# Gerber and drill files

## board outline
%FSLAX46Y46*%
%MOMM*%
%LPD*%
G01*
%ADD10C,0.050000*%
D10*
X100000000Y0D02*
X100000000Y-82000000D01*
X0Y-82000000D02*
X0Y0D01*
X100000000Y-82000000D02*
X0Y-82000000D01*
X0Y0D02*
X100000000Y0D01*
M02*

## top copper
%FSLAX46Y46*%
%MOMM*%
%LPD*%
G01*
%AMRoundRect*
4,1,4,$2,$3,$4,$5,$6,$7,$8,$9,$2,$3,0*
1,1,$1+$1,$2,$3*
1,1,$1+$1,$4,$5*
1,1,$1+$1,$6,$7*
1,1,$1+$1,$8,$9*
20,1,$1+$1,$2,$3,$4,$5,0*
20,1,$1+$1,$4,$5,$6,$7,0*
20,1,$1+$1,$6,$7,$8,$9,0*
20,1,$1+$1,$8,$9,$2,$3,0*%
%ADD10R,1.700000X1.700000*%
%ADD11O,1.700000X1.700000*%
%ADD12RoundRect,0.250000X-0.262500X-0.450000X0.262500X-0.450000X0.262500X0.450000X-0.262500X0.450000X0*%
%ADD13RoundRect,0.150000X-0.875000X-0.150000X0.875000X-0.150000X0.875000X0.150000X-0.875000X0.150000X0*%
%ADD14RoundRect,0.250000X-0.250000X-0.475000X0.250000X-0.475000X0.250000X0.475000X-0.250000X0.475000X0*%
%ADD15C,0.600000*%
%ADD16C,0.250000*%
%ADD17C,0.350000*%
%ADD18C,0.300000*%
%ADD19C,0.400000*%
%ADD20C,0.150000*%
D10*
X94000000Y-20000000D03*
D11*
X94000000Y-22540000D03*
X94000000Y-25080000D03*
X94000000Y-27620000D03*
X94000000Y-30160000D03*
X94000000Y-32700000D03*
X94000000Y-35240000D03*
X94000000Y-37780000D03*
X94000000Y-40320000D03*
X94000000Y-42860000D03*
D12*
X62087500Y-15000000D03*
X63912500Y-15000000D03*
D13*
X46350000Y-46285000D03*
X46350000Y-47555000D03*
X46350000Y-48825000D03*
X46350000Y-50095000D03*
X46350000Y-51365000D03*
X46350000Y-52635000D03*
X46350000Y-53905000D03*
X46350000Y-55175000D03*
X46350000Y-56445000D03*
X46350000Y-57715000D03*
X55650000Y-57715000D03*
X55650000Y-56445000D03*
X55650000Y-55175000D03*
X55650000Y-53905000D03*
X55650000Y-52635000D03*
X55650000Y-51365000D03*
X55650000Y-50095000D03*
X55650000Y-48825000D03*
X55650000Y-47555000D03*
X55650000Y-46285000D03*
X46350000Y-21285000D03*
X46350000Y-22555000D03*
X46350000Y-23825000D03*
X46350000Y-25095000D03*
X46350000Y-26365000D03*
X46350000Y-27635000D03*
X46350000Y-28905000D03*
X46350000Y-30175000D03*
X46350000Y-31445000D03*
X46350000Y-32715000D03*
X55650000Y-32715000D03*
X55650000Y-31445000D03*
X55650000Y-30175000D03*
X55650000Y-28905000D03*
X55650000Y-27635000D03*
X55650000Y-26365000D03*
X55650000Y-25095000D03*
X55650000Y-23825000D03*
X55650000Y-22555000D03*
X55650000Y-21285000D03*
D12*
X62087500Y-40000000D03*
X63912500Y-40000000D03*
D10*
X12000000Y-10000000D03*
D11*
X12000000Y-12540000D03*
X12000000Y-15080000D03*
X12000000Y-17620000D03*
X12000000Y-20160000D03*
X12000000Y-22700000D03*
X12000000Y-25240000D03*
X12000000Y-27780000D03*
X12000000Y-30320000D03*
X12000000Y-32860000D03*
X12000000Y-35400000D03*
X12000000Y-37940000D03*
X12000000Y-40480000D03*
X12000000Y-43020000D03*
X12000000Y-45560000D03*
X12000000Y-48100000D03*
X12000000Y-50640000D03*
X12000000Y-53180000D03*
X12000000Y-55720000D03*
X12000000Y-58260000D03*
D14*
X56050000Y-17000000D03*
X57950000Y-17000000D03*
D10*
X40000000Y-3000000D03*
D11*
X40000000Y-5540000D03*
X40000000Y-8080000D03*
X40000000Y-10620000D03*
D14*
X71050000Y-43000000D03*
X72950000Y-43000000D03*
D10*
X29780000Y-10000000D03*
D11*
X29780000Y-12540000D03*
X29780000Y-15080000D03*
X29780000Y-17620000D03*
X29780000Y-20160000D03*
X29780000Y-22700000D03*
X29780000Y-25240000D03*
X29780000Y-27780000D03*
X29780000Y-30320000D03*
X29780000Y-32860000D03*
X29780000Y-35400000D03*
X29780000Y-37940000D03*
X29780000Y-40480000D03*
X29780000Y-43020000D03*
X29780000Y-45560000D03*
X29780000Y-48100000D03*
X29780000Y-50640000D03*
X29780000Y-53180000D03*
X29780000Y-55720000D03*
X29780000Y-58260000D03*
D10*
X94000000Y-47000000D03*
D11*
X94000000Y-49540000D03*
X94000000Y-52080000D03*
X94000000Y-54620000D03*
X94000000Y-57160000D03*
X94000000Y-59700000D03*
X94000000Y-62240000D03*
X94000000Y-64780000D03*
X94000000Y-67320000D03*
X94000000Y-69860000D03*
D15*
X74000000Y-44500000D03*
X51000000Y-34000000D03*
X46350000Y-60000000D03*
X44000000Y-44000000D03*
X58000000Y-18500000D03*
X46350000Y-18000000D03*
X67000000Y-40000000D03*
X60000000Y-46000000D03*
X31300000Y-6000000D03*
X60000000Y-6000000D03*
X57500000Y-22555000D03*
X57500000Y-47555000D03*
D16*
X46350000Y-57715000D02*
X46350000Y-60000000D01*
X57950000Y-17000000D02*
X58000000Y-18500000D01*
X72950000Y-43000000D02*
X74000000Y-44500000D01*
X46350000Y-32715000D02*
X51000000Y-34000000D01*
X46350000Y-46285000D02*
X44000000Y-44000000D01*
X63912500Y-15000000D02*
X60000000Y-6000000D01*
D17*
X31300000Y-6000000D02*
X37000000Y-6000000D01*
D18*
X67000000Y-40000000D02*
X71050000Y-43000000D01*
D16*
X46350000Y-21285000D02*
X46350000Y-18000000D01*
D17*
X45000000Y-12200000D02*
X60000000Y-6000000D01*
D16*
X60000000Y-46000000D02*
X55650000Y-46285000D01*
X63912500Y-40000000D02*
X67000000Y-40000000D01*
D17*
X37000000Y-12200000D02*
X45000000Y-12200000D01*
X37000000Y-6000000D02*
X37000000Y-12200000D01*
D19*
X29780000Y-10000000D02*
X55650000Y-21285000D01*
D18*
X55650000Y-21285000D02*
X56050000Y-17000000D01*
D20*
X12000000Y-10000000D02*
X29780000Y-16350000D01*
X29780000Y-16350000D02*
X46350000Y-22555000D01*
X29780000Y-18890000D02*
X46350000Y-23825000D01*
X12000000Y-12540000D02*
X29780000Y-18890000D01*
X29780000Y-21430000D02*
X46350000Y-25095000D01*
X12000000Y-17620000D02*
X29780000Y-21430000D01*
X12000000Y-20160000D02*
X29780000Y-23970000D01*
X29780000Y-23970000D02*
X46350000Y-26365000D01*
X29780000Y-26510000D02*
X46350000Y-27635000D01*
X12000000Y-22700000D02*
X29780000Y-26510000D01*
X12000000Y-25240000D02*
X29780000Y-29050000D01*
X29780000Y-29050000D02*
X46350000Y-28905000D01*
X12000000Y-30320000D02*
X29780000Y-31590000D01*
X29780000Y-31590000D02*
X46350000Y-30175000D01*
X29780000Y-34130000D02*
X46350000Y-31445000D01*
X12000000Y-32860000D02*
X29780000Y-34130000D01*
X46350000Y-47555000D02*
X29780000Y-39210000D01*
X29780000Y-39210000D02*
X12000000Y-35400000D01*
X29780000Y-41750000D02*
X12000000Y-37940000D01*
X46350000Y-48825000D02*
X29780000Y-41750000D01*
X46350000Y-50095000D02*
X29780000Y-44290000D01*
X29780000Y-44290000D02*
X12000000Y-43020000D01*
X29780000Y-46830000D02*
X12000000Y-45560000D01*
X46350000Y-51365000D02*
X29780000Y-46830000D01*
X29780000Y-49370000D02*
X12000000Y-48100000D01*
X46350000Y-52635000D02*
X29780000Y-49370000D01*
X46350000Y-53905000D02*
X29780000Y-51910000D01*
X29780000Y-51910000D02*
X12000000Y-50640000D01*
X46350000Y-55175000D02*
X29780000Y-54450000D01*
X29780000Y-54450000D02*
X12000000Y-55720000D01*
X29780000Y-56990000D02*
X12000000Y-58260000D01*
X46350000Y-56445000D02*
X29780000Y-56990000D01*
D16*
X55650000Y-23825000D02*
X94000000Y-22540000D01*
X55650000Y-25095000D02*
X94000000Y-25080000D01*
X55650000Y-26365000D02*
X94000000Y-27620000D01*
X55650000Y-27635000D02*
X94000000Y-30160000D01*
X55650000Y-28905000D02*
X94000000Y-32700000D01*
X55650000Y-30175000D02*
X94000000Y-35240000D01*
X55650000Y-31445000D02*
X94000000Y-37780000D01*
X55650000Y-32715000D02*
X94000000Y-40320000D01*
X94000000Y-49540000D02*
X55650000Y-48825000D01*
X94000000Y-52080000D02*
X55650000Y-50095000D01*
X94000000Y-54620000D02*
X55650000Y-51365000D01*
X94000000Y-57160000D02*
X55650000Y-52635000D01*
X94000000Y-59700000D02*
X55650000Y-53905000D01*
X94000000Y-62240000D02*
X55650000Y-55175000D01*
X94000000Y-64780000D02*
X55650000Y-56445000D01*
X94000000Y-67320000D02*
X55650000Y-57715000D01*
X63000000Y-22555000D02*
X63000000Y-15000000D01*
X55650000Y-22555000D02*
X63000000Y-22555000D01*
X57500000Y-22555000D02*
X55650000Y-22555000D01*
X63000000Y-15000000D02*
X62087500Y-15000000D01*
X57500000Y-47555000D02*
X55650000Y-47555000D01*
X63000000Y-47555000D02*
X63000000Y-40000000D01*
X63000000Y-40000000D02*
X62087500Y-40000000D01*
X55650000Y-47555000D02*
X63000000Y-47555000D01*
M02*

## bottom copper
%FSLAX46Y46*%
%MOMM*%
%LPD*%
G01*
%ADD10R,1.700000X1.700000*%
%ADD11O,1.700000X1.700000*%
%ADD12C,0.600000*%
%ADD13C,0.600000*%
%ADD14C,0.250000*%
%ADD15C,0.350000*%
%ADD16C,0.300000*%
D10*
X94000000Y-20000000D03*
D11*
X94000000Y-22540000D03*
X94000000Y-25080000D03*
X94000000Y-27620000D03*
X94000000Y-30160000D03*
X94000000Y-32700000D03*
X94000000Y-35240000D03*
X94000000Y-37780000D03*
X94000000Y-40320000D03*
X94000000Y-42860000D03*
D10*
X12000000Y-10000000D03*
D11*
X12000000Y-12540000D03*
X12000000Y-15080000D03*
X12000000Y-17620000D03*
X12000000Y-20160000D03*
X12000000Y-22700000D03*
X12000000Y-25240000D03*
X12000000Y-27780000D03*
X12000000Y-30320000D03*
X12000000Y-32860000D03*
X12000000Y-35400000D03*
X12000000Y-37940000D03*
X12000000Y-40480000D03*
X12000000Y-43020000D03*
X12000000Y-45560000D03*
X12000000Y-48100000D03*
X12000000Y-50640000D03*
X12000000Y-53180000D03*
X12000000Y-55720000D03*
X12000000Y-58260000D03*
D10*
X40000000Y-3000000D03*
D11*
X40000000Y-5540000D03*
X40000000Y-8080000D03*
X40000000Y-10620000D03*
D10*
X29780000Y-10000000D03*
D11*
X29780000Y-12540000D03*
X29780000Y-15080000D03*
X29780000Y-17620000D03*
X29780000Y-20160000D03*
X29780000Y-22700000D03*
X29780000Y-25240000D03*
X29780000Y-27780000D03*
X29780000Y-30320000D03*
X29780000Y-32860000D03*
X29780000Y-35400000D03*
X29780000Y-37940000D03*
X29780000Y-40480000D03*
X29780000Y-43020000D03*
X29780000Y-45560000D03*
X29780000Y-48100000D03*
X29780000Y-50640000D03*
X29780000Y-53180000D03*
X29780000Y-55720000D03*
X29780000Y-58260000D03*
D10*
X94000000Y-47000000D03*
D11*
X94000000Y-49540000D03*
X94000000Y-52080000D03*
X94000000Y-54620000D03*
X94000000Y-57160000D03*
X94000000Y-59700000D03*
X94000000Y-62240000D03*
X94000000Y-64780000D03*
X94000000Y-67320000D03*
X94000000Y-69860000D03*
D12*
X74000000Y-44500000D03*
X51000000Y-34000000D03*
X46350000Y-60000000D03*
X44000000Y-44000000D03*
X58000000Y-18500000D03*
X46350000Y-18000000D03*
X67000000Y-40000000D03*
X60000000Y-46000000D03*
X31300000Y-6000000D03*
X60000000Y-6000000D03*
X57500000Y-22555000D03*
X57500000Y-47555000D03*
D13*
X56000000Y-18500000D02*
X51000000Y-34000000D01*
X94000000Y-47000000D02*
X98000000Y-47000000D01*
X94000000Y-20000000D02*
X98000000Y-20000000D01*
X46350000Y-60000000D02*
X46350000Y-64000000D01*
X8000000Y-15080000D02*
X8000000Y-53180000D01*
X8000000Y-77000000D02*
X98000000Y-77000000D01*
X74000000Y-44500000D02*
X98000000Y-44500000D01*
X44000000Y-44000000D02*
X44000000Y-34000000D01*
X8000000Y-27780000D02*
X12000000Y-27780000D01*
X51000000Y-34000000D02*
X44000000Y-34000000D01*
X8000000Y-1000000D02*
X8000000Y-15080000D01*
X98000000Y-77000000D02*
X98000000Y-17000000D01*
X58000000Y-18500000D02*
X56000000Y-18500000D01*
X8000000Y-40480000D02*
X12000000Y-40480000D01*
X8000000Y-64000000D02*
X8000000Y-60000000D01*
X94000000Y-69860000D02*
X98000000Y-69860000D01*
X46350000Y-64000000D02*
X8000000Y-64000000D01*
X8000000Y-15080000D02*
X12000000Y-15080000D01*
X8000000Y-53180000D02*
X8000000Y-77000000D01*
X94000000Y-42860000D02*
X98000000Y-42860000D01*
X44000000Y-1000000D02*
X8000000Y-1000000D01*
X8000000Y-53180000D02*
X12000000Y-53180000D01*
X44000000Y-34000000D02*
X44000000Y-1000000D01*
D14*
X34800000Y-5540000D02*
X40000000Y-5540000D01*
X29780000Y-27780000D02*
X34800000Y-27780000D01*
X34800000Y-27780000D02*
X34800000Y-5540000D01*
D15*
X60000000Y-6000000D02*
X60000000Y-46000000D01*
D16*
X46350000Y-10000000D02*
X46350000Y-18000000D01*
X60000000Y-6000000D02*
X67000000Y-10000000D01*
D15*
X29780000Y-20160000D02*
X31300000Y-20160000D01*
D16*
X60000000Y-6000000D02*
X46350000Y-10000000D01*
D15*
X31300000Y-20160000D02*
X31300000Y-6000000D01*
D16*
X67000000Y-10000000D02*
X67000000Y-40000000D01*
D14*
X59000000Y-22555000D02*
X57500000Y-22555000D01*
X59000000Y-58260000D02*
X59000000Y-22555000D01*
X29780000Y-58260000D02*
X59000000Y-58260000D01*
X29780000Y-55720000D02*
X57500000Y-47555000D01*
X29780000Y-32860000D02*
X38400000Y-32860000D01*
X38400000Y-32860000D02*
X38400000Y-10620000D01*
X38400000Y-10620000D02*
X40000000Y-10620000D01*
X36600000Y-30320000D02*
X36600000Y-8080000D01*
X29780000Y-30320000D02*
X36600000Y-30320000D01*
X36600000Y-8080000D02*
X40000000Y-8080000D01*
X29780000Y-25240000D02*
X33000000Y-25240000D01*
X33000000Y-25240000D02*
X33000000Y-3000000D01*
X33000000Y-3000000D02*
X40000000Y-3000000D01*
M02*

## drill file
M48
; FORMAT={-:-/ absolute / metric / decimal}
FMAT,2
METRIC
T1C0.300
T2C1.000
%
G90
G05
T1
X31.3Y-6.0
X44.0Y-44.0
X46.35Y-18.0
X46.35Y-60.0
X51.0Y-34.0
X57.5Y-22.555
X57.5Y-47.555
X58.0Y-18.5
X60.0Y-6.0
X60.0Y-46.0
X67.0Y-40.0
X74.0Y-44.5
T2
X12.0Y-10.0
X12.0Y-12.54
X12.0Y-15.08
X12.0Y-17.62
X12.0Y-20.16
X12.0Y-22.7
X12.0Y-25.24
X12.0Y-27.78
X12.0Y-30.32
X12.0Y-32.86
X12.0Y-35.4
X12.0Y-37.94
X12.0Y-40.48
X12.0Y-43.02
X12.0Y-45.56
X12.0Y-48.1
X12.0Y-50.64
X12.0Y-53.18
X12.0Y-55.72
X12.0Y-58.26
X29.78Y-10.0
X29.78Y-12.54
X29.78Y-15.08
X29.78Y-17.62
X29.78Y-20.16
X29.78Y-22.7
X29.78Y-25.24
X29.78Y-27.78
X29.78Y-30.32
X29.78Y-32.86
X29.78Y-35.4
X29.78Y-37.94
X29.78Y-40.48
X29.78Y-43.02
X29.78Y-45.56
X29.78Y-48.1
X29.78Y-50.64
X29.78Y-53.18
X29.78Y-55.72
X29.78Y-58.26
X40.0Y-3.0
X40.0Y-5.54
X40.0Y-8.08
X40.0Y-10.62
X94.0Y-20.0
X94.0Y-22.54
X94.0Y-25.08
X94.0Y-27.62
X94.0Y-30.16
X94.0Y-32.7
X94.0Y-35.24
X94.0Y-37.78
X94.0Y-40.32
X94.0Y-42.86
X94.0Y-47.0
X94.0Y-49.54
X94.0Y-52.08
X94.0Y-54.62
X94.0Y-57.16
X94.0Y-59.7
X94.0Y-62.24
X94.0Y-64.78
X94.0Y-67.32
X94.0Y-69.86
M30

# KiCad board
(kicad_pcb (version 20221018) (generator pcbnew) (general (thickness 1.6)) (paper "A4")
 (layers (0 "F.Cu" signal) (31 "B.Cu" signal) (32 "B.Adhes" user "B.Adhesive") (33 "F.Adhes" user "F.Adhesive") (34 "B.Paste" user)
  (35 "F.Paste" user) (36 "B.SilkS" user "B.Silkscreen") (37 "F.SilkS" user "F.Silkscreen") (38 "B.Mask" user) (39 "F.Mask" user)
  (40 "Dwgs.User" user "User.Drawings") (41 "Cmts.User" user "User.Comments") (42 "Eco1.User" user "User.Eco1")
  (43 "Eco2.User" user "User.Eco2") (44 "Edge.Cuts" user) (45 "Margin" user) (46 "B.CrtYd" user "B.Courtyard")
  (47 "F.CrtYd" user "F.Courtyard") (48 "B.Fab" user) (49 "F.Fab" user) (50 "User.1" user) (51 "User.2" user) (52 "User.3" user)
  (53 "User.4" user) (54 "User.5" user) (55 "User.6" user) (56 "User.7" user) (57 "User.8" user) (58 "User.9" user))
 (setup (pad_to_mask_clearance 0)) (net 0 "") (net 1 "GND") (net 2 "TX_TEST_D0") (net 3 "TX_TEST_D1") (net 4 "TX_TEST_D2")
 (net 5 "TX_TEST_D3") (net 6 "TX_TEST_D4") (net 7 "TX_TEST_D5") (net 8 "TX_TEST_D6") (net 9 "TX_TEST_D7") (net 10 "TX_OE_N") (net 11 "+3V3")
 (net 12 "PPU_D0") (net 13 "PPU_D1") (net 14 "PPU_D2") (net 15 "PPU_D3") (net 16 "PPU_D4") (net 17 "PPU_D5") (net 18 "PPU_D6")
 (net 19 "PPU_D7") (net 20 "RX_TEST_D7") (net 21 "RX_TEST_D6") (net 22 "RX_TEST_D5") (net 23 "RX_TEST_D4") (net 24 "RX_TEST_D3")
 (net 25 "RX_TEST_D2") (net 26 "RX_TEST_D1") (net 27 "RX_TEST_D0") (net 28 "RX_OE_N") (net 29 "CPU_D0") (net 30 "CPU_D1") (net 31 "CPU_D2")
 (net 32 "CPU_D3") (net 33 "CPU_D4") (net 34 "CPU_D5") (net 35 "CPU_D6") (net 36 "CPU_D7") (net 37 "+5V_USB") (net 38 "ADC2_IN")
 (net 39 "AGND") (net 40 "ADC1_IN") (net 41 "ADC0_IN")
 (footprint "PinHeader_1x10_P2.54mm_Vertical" (layer "F.Cu") (at 94 20)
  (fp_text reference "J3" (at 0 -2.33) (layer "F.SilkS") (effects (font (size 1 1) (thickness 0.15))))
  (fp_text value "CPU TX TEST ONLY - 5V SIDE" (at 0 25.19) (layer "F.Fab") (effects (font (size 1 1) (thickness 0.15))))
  (pad "1" thru_hole rect (at 0 0) (size 1.7 1.7) (drill 1) (layers "*.Cu" "*.Mask") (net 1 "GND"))
  (pad "2" thru_hole oval (at 0 2.54) (size 1.7 1.7) (drill 1) (layers "*.Cu" "*.Mask") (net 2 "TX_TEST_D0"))
  (pad "3" thru_hole oval (at 0 5.08) (size 1.7 1.7) (drill 1) (layers "*.Cu" "*.Mask") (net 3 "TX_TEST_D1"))
  (pad "4" thru_hole oval (at 0 7.62) (size 1.7 1.7) (drill 1) (layers "*.Cu" "*.Mask") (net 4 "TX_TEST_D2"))
  (pad "5" thru_hole oval (at 0 10.16) (size 1.7 1.7) (drill 1) (layers "*.Cu" "*.Mask") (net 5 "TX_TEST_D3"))
  (pad "6" thru_hole oval (at 0 12.7) (size 1.7 1.7) (drill 1) (layers "*.Cu" "*.Mask") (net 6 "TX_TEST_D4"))
  (pad "7" thru_hole oval (at 0 15.24) (size 1.7 1.7) (drill 1) (layers "*.Cu" "*.Mask") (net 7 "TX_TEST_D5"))
  (pad "8" thru_hole oval (at 0 17.78) (size 1.7 1.7) (drill 1) (layers "*.Cu" "*.Mask") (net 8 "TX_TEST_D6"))
  (pad "9" thru_hole oval (at 0 20.32) (size 1.7 1.7) (drill 1) (layers "*.Cu" "*.Mask") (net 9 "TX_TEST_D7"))
  (pad "10" thru_hole oval (at 0 22.86) (size 1.7 1.7) (drill 1) (layers "*.Cu" "*.Mask") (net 1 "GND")))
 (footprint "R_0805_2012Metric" (layer "F.Cu") (at 63 15)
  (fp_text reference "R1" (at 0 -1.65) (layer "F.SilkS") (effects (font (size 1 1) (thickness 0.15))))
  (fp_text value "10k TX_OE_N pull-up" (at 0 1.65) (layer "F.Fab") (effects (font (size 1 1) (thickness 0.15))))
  (pad "1" smd roundrect (at -0.9125 0) (size 1.025 1.4) (layers "F.Cu" "F.Paste" "F.Mask") (roundrect_rratio 0.243902) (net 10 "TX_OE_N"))
  (pad "2" smd roundrect (at 0.9125 0) (size 1.025 1.4) (layers "F.Cu" "F.Paste" "F.Mask") (roundrect_rratio 0.243902) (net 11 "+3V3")))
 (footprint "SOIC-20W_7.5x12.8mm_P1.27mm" (layer "F.Cu") (at 51 52)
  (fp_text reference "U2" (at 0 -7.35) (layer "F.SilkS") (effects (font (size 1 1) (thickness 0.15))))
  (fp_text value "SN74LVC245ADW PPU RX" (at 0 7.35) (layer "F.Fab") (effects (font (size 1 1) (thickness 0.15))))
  (pad "1" smd roundrect (at -4.65 -5.715) (size 2.05 0.6) (layers "F.Cu" "F.Paste" "F.Mask") (roundrect_rratio 0.25) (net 1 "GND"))
  (pad "2" smd roundrect (at -4.65 -4.445) (size 2.05 0.6) (layers "F.Cu" "F.Paste" "F.Mask") (roundrect_rratio 0.25) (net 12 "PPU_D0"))
  (pad "3" smd roundrect (at -4.65 -3.175) (size 2.05 0.6) (layers "F.Cu" "F.Paste" "F.Mask") (roundrect_rratio 0.25) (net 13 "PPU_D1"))
  (pad "4" smd roundrect (at -4.65 -1.905) (size 2.05 0.6) (layers "F.Cu" "F.Paste" "F.Mask") (roundrect_rratio 0.25) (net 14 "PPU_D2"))
  (pad "5" smd roundrect (at -4.65 -0.635) (size 2.05 0.6) (layers "F.Cu" "F.Paste" "F.Mask") (roundrect_rratio 0.25) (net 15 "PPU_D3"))
  (pad "6" smd roundrect (at -4.65 0.635) (size 2.05 0.6) (layers "F.Cu" "F.Paste" "F.Mask") (roundrect_rratio 0.25) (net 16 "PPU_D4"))
  (pad "7" smd roundrect (at -4.65 1.905) (size 2.05 0.6) (layers "F.Cu" "F.Paste" "F.Mask") (roundrect_rratio 0.25) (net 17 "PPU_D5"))
  (pad "8" smd roundrect (at -4.65 3.175) (size 2.05 0.6) (layers "F.Cu" "F.Paste" "F.Mask") (roundrect_rratio 0.25) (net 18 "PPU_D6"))
  (pad "9" smd roundrect (at -4.65 4.445) (size 2.05 0.6) (layers "F.Cu" "F.Paste" "F.Mask") (roundrect_rratio 0.25) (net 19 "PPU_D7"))
  (pad "10" smd roundrect (at -4.65 5.715) (size 2.05 0.6) (layers "F.Cu" "F.Paste" "F.Mask") (roundrect_rratio 0.25) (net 1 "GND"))
  (pad "11" smd roundrect (at 4.65 5.715) (size 2.05 0.6) (layers "F.Cu" "F.Paste" "F.Mask") (roundrect_rratio 0.25) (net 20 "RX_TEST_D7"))
  (pad "12" smd roundrect (at 4.65 4.445) (size 2.05 0.6) (layers "F.Cu" "F.Paste" "F.Mask") (roundrect_rratio 0.25) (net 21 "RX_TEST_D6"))
  (pad "13" smd roundrect (at 4.65 3.175) (size 2.05 0.6) (layers "F.Cu" "F.Paste" "F.Mask") (roundrect_rratio 0.25) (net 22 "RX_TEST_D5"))
  (pad "14" smd roundrect (at 4.65 1.905) (size 2.05 0.6) (layers "F.Cu" "F.Paste" "F.Mask") (roundrect_rratio 0.25) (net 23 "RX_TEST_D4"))
  (pad "15" smd roundrect (at 4.65 0.635) (size 2.05 0.6) (layers "F.Cu" "F.Paste" "F.Mask") (roundrect_rratio 0.25) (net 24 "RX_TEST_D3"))
  (pad "16" smd roundrect (at 4.65 -0.635) (size 2.05 0.6) (layers "F.Cu" "F.Paste" "F.Mask") (roundrect_rratio 0.25) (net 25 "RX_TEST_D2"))
  (pad "17" smd roundrect (at 4.65 -1.905) (size 2.05 0.6) (layers "F.Cu" "F.Paste" "F.Mask") (roundrect_rratio 0.25) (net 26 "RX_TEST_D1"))
  (pad "18" smd roundrect (at 4.65 -3.175) (size 2.05 0.6) (layers "F.Cu" "F.Paste" "F.Mask") (roundrect_rratio 0.25) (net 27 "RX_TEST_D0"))
  (pad "19" smd roundrect (at 4.65 -4.445) (size 2.05 0.6) (layers "F.Cu" "F.Paste" "F.Mask") (roundrect_rratio 0.25) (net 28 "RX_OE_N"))
  (pad "20" smd roundrect (at 4.65 -5.715) (size 2.05 0.6) (layers "F.Cu" "F.Paste" "F.Mask") (roundrect_rratio 0.25) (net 11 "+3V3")))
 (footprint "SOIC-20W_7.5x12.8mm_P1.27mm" (layer "F.Cu") (at 51 27)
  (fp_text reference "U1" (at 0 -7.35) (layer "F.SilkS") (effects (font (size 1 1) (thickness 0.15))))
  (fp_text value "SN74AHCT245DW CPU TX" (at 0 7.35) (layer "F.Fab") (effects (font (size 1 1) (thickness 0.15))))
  (pad "1" smd roundrect (at -4.65 -5.715) (size 2.05 0.6) (layers "F.Cu" "F.Paste" "F.Mask") (roundrect_rratio 0.25) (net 11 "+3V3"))
  (pad "2" smd roundrect (at -4.65 -4.445) (size 2.05 0.6) (layers "F.Cu" "F.Paste" "F.Mask") (roundrect_rratio 0.25) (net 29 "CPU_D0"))
  (pad "3" smd roundrect (at -4.65 -3.175) (size 2.05 0.6) (layers "F.Cu" "F.Paste" "F.Mask") (roundrect_rratio 0.25) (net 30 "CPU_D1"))
  (pad "4" smd roundrect (at -4.65 -1.905) (size 2.05 0.6) (layers "F.Cu" "F.Paste" "F.Mask") (roundrect_rratio 0.25) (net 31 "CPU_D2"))
  (pad "5" smd roundrect (at -4.65 -0.635) (size 2.05 0.6) (layers "F.Cu" "F.Paste" "F.Mask") (roundrect_rratio 0.25) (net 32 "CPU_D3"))
  (pad "6" smd roundrect (at -4.65 0.635) (size 2.05 0.6) (layers "F.Cu" "F.Paste" "F.Mask") (roundrect_rratio 0.25) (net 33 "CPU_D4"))
  (pad "7" smd roundrect (at -4.65 1.905) (size 2.05 0.6) (layers "F.Cu" "F.Paste" "F.Mask") (roundrect_rratio 0.25) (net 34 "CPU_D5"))
  (pad "8" smd roundrect (at -4.65 3.175) (size 2.05 0.6) (layers "F.Cu" "F.Paste" "F.Mask") (roundrect_rratio 0.25) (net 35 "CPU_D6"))
  (pad "9" smd roundrect (at -4.65 4.445) (size 2.05 0.6) (layers "F.Cu" "F.Paste" "F.Mask") (roundrect_rratio 0.25) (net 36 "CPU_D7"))
  (pad "10" smd roundrect (at -4.65 5.715) (size 2.05 0.6) (layers "F.Cu" "F.Paste" "F.Mask") (roundrect_rratio 0.25) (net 1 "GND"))
  (pad "11" smd roundrect (at 4.65 5.715) (size 2.05 0.6) (layers "F.Cu" "F.Paste" "F.Mask") (roundrect_rratio 0.25) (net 9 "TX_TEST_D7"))
  (pad "12" smd roundrect (at 4.65 4.445) (size 2.05 0.6) (layers "F.Cu" "F.Paste" "F.Mask") (roundrect_rratio 0.25) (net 8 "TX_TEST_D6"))
  (pad "13" smd roundrect (at 4.65 3.175) (size 2.05 0.6) (layers "F.Cu" "F.Paste" "F.Mask") (roundrect_rratio 0.25) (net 7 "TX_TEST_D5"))
  (pad "14" smd roundrect (at 4.65 1.905) (size 2.05 0.6) (layers "F.Cu" "F.Paste" "F.Mask") (roundrect_rratio 0.25) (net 6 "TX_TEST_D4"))
  (pad "15" smd roundrect (at 4.65 0.635) (size 2.05 0.6) (layers "F.Cu" "F.Paste" "F.Mask") (roundrect_rratio 0.25) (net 5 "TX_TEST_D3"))
  (pad "16" smd roundrect (at 4.65 -0.635) (size 2.05 0.6) (layers "F.Cu" "F.Paste" "F.Mask") (roundrect_rratio 0.25) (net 4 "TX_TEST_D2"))
  (pad "17" smd roundrect (at 4.65 -1.905) (size 2.05 0.6) (layers "F.Cu" "F.Paste" "F.Mask") (roundrect_rratio 0.25) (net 3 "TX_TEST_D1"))
  (pad "18" smd roundrect (at 4.65 -3.175) (size 2.05 0.6) (layers "F.Cu" "F.Paste" "F.Mask") (roundrect_rratio 0.25) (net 2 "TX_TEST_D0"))
  (pad "19" smd roundrect (at 4.65 -4.445) (size 2.05 0.6) (layers "F.Cu" "F.Paste" "F.Mask") (roundrect_rratio 0.25) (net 10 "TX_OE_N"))
  (pad "20" smd roundrect (at 4.65 -5.715) (size 2.05 0.6) (layers "F.Cu" "F.Paste" "F.Mask") (roundrect_rratio 0.25) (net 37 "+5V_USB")))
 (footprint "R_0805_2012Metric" (layer "F.Cu") (at 63 40)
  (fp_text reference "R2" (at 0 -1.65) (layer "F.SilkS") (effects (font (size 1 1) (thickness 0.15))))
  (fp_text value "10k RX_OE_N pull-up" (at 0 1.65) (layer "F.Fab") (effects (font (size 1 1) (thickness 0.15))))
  (pad "1" smd roundrect (at -0.9125 0) (size 1.025 1.4) (layers "F.Cu" "F.Paste" "F.Mask") (roundrect_rratio 0.243902) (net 28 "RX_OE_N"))
  (pad "2" smd roundrect (at 0.9125 0) (size 1.025 1.4) (layers "F.Cu" "F.Paste" "F.Mask") (roundrect_rratio 0.243902) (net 11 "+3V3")))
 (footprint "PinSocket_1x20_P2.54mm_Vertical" (layer "F.Cu") (at 12 10)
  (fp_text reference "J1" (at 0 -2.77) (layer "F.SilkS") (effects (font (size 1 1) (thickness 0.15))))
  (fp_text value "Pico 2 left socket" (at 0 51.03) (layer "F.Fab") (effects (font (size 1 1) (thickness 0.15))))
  (pad "1" thru_hole rect (at 0 0) (size 1.7 1.7) (drill 1) (layers "*.Cu" "*.Mask") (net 29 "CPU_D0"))
  (pad "2" thru_hole oval (at 0 2.54) (size 1.7 1.7) (drill 1) (layers "*.Cu" "*.Mask") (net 30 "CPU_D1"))
  (pad "3" thru_hole oval (at 0 5.08) (size 1.7 1.7) (drill 1) (layers "*.Cu" "*.Mask") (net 1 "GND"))
  (pad "4" thru_hole oval (at 0 7.62) (size 1.7 1.7) (drill 1) (layers "*.Cu" "*.Mask") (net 31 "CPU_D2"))
  (pad "5" thru_hole oval (at 0 10.16) (size 1.7 1.7) (drill 1) (layers "*.Cu" "*.Mask") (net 32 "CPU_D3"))
  (pad "6" thru_hole oval (at 0 12.7) (size 1.7 1.7) (drill 1) (layers "*.Cu" "*.Mask") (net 33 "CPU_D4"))
  (pad "7" thru_hole oval (at 0 15.24) (size 1.7 1.7) (drill 1) (layers "*.Cu" "*.Mask") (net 34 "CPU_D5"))
  (pad "8" thru_hole oval (at 0 17.78) (size 1.7 1.7) (drill 1) (layers "*.Cu" "*.Mask") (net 1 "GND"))
  (pad "9" thru_hole oval (at 0 20.32) (size 1.7 1.7) (drill 1) (layers "*.Cu" "*.Mask") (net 35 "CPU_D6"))
  (pad "10" thru_hole oval (at 0 22.86) (size 1.7 1.7) (drill 1) (layers "*.Cu" "*.Mask") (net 36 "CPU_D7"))
  (pad "11" thru_hole oval (at 0 25.4) (size 1.7 1.7) (drill 1) (layers "*.Cu" "*.Mask") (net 12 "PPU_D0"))
  (pad "12" thru_hole oval (at 0 27.94) (size 1.7 1.7) (drill 1) (layers "*.Cu" "*.Mask") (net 13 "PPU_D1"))
  (pad "13" thru_hole oval (at 0 30.48) (size 1.7 1.7) (drill 1) (layers "*.Cu" "*.Mask") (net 1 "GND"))
  (pad "14" thru_hole oval (at 0 33.02) (size 1.7 1.7) (drill 1) (layers "*.Cu" "*.Mask") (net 14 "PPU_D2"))
  (pad "15" thru_hole oval (at 0 35.56) (size 1.7 1.7) (drill 1) (layers "*.Cu" "*.Mask") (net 15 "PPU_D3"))
  (pad "16" thru_hole oval (at 0 38.1) (size 1.7 1.7) (drill 1) (layers "*.Cu" "*.Mask") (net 16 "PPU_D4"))
  (pad "17" thru_hole oval (at 0 40.64) (size 1.7 1.7) (drill 1) (layers "*.Cu" "*.Mask") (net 17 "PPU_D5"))
  (pad "18" thru_hole oval (at 0 43.18) (size 1.7 1.7) (drill 1) (layers "*.Cu" "*.Mask") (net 1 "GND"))
  (pad "19" thru_hole oval (at 0 45.72) (size 1.7 1.7) (drill 1) (layers "*.Cu" "*.Mask") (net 18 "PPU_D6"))
  (pad "20" thru_hole oval (at 0 48.26) (size 1.7 1.7) (drill 1) (layers "*.Cu" "*.Mask") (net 19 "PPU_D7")))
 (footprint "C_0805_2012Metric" (layer "F.Cu") (at 57 17)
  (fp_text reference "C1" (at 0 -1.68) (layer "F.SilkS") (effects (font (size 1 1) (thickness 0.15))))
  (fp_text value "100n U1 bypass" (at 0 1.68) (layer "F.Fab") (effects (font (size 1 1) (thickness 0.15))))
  (pad "1" smd roundrect (at -0.95 0) (size 1 1.45) (layers "F.Cu" "F.Paste" "F.Mask") (roundrect_rratio 0.25) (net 37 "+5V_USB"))
  (pad "2" smd roundrect (at 0.95 0) (size 1 1.45) (layers "F.Cu" "F.Paste" "F.Mask") (roundrect_rratio 0.25) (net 1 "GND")))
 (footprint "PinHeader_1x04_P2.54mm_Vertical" (layer "F.Cu") (at 40 3)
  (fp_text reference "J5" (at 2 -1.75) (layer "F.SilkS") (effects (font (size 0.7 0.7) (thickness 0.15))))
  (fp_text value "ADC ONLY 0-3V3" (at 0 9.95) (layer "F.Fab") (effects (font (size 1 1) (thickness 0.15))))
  (pad "1" thru_hole rect (at 0 0) (size 1.7 1.7) (drill 1) (layers "*.Cu" "*.Mask") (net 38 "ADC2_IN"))
  (pad "2" thru_hole oval (at 0 2.54) (size 1.7 1.7) (drill 1) (layers "*.Cu" "*.Mask") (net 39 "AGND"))
  (pad "3" thru_hole oval (at 0 5.08) (size 1.7 1.7) (drill 1) (layers "*.Cu" "*.Mask") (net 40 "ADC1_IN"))
  (pad "4" thru_hole oval (at 0 7.62) (size 1.7 1.7) (drill 1) (layers "*.Cu" "*.Mask") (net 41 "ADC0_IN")))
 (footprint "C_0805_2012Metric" (layer "F.Cu") (at 72 43)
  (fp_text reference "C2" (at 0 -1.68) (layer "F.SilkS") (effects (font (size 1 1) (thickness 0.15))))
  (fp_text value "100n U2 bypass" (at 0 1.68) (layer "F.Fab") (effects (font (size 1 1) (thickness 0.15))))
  (pad "1" smd roundrect (at -0.95 0) (size 1 1.45) (layers "F.Cu" "F.Paste" "F.Mask") (roundrect_rratio 0.25) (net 11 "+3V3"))
  (pad "2" smd roundrect (at 0.95 0) (size 1 1.45) (layers "F.Cu" "F.Paste" "F.Mask") (roundrect_rratio 0.25) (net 1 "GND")))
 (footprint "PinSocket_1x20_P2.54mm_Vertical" (layer "F.Cu") (at 29.78 10)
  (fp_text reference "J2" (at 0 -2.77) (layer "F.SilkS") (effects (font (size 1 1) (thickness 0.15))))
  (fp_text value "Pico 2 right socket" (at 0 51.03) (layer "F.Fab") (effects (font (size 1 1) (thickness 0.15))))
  (pad "1" thru_hole rect (at 0 0) (size 1.7 1.7) (drill 1) (layers "*.Cu" "*.Mask") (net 37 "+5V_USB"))
  (pad "2" thru_hole oval (at 0 2.54) (size 1.7 1.7) (drill 1) (layers "*.Cu" "*.Mask"))
  (pad "3" thru_hole oval (at 0 5.08) (size 1.7 1.7) (drill 1) (layers "*.Cu" "*.Mask"))
  (pad "4" thru_hole oval (at 0 7.62) (size 1.7 1.7) (drill 1) (layers "*.Cu" "*.Mask"))
  (pad "5" thru_hole oval (at 0 10.16) (size 1.7 1.7) (drill 1) (layers "*.Cu" "*.Mask") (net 11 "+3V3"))
  (pad "6" thru_hole oval (at 0 12.7) (size 1.7 1.7) (drill 1) (layers "*.Cu" "*.Mask"))
  (pad "7" thru_hole oval (at 0 15.24) (size 1.7 1.7) (drill 1) (layers "*.Cu" "*.Mask") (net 38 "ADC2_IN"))
  (pad "8" thru_hole oval (at 0 17.78) (size 1.7 1.7) (drill 1) (layers "*.Cu" "*.Mask") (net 39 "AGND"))
  (pad "9" thru_hole oval (at 0 20.32) (size 1.7 1.7) (drill 1) (layers "*.Cu" "*.Mask") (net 40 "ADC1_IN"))
  (pad "10" thru_hole oval (at 0 22.86) (size 1.7 1.7) (drill 1) (layers "*.Cu" "*.Mask") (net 41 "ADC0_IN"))
  (pad "11" thru_hole oval (at 0 25.4) (size 1.7 1.7) (drill 1) (layers "*.Cu" "*.Mask"))
  (pad "12" thru_hole oval (at 0 27.94) (size 1.7 1.7) (drill 1) (layers "*.Cu" "*.Mask"))
  (pad "13" thru_hole oval (at 0 30.48) (size 1.7 1.7) (drill 1) (layers "*.Cu" "*.Mask"))
  (pad "14" thru_hole oval (at 0 33.02) (size 1.7 1.7) (drill 1) (layers "*.Cu" "*.Mask"))
  (pad "15" thru_hole oval (at 0 35.56) (size 1.7 1.7) (drill 1) (layers "*.Cu" "*.Mask"))
  (pad "16" thru_hole oval (at 0 38.1) (size 1.7 1.7) (drill 1) (layers "*.Cu" "*.Mask"))
  (pad "17" thru_hole oval (at 0 40.64) (size 1.7 1.7) (drill 1) (layers "*.Cu" "*.Mask"))
  (pad "18" thru_hole oval (at 0 43.18) (size 1.7 1.7) (drill 1) (layers "*.Cu" "*.Mask"))
  (pad "19" thru_hole oval (at 0 45.72) (size 1.7 1.7) (drill 1) (layers "*.Cu" "*.Mask") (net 28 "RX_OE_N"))
  (pad "20" thru_hole oval (at 0 48.26) (size 1.7 1.7) (drill 1) (layers "*.Cu" "*.Mask") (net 10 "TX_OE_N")))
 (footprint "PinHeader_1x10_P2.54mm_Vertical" (layer "F.Cu") (at 94 47)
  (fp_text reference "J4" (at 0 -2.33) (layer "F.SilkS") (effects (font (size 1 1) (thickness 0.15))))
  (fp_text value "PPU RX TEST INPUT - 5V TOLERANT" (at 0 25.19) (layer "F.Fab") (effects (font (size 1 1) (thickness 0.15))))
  (pad "1" thru_hole rect (at 0 0) (size 1.7 1.7) (drill 1) (layers "*.Cu" "*.Mask") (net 1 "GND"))
  (pad "2" thru_hole oval (at 0 2.54) (size 1.7 1.7) (drill 1) (layers "*.Cu" "*.Mask") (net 27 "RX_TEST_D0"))
  (pad "3" thru_hole oval (at 0 5.08) (size 1.7 1.7) (drill 1) (layers "*.Cu" "*.Mask") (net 26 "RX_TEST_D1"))
  (pad "4" thru_hole oval (at 0 7.62) (size 1.7 1.7) (drill 1) (layers "*.Cu" "*.Mask") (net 25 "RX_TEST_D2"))
  (pad "5" thru_hole oval (at 0 10.16) (size 1.7 1.7) (drill 1) (layers "*.Cu" "*.Mask") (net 24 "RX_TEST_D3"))
  (pad "6" thru_hole oval (at 0 12.7) (size 1.7 1.7) (drill 1) (layers "*.Cu" "*.Mask") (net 23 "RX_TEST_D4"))
  (pad "7" thru_hole oval (at 0 15.24) (size 1.7 1.7) (drill 1) (layers "*.Cu" "*.Mask") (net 22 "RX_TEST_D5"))
  (pad "8" thru_hole oval (at 0 17.78) (size 1.7 1.7) (drill 1) (layers "*.Cu" "*.Mask") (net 21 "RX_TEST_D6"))
  (pad "9" thru_hole oval (at 0 20.32) (size 1.7 1.7) (drill 1) (layers "*.Cu" "*.Mask") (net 20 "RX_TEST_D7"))
  (pad "10" thru_hole oval (at 0 22.86) (size 1.7 1.7) (drill 1) (layers "*.Cu" "*.Mask") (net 1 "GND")))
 (gr_line (start 100 0) (end 100 82) (stroke (width 0.05) (type default)) (layer "Edge.Cuts"))
 (gr_line (start 0 82) (end 0 0) (stroke (width 0.05) (type default)) (layer "Edge.Cuts"))
 (gr_line (start 100 82) (end 0 82) (stroke (width 0.05) (type default)) (layer "Edge.Cuts"))
 (gr_line (start 0 0) (end 100 0) (stroke (width 0.05) (type default)) (layer "Edge.Cuts"))
 (segment (start 46.35 57.715) (end 46.35 60) (width 0.25) (layer "F.Cu") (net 1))
 (segment (start 57.95 17) (end 58 18.5) (width 0.25) (layer "F.Cu") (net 1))
 (segment (start 72.95 43) (end 74 44.5) (width 0.25) (layer "F.Cu") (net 1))
 (segment (start 46.35 32.715) (end 51 34) (width 0.25) (layer "F.Cu") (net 1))
 (segment (start 46.35 46.285) (end 44 44) (width 0.25) (layer "F.Cu") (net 1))
 (via (at 74 44.5) (size 0.6) (drill 0.3) (layers "F.Cu" "B.Cu") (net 1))
 (via (at 51 34) (size 0.6) (drill 0.3) (layers "F.Cu" "B.Cu") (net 1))
 (via (at 46.35 60) (size 0.6) (drill 0.3) (layers "F.Cu" "B.Cu") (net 1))
 (via (at 44 44) (size 0.6) (drill 0.3) (layers "F.Cu" "B.Cu") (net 1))
 (via (at 58 18.5) (size 0.6) (drill 0.3) (layers "F.Cu" "B.Cu") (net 1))
 (segment (start 56 18.5) (end 51 34) (width 0.6) (layer "B.Cu") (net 1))
 (segment (start 94 47) (end 98 47) (width 0.6) (layer "B.Cu") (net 1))
 (segment (start 94 20) (end 98 20) (width 0.6) (layer "B.Cu") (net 1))
 (segment (start 46.35 60) (end 46.35 64) (width 0.6) (layer "B.Cu") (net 1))
 (segment (start 8 15.08) (end 8 53.18) (width 0.6) (layer "B.Cu") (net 1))
 (segment (start 8 77) (end 98 77) (width 0.6) (layer "B.Cu") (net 1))
 (segment (start 74 44.5) (end 98 44.5) (width 0.6) (layer "B.Cu") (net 1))
 (segment (start 44 44) (end 44 34) (width 0.6) (layer "B.Cu") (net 1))
 (segment (start 8 27.78) (end 12 27.78) (width 0.6) (layer "B.Cu") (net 1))
 (segment (start 51 34) (end 44 34) (width 0.6) (layer "B.Cu") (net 1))
 (segment (start 8 1) (end 8 15.08) (width 0.6) (layer "B.Cu") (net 1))
 (segment (start 98 77) (end 98 17) (width 0.6) (layer "B.Cu") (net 1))
 (segment (start 58 18.5) (end 56 18.5) (width 0.6) (layer "B.Cu") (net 1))
 (segment (start 8 40.48) (end 12 40.48) (width 0.6) (layer "B.Cu") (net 1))
 (segment (start 8 64) (end 8 60) (width 0.6) (layer "B.Cu") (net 1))
 (segment (start 94 69.86) (end 98 69.86) (width 0.6) (layer "B.Cu") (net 1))
 (segment (start 46.35 64) (end 8 64) (width 0.6) (layer "B.Cu") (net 1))
 (segment (start 8 15.08) (end 12 15.08) (width 0.6) (layer "B.Cu") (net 1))
 (segment (start 8 53.18) (end 8 77) (width 0.6) (layer "B.Cu") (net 1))
 (segment (start 94 42.86) (end 98 42.86) (width 0.6) (layer "B.Cu") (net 1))
 (segment (start 44 1) (end 8 1) (width 0.6) (layer "B.Cu") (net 1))
 (segment (start 8 53.18) (end 12 53.18) (width 0.6) (layer "B.Cu") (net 1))
 (segment (start 44 34) (end 44 1) (width 0.6) (layer "B.Cu") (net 1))
 (segment (start 34.8 5.54) (end 40 5.54) (width 0.25) (layer "B.Cu") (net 39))
 (segment (start 29.78 27.78) (end 34.8 27.78) (width 0.25) (layer "B.Cu") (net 39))
 (segment (start 34.8 27.78) (end 34.8 5.54) (width 0.25) (layer "B.Cu") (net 39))
 (segment (start 63.9125 15) (end 60 6) (width 0.25) (layer "F.Cu") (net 11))
 (segment (start 31.3 6) (end 37 6) (width 0.35) (layer "F.Cu") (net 11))
 (segment (start 67 40) (end 71.05 43) (width 0.3) (layer "F.Cu") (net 11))
 (segment (start 46.35 21.285) (end 46.35 18) (width 0.25) (layer "F.Cu") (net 11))
 (segment (start 45 12.2) (end 60 6) (width 0.35) (layer "F.Cu") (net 11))
 (segment (start 60 46) (end 55.65 46.285) (width 0.25) (layer "F.Cu") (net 11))
 (segment (start 63.9125 40) (end 67 40) (width 0.25) (layer "F.Cu") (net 11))
 (segment (start 37 12.2) (end 45 12.2) (width 0.35) (layer "F.Cu") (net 11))
 (segment (start 37 6) (end 37 12.2) (width 0.35) (layer "F.Cu") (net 11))
 (via (at 46.35 18) (size 0.6) (drill 0.3) (layers "F.Cu" "B.Cu") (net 11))
 (via (at 67 40) (size 0.6) (drill 0.3) (layers "F.Cu" "B.Cu") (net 11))
 (via (at 60 46) (size 0.6) (drill 0.3) (layers "F.Cu" "B.Cu") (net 11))
 (via (at 31.3 6) (size 0.6) (drill 0.3) (layers "F.Cu" "B.Cu") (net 11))
 (via (at 60 6) (size 0.6) (drill 0.3) (layers "F.Cu" "B.Cu") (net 11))
 (segment (start 60 6) (end 60 46) (width 0.35) (layer "B.Cu") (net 11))
 (segment (start 46.35 10) (end 46.35 18) (width 0.3) (layer "B.Cu") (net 11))
 (segment (start 60 6) (end 67 10) (width 0.3) (layer "B.Cu") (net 11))
 (segment (start 29.78 20.16) (end 31.3 20.16) (width 0.35) (layer "B.Cu") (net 11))
 (segment (start 60 6) (end 46.35 10) (width 0.3) (layer "B.Cu") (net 11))
 (segment (start 31.3 20.16) (end 31.3 6) (width 0.35) (layer "B.Cu") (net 11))
 (segment (start 67 10) (end 67 40) (width 0.3) (layer "B.Cu") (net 11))
 (segment (start 29.78 10) (end 55.65 21.285) (width 0.4) (layer "F.Cu") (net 37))
 (segment (start 55.65 21.285) (end 56.05 17) (width 0.3) (layer "F.Cu") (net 37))
 (segment (start 12 10) (end 29.78 16.35) (width 0.15) (layer "F.Cu") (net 29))
 (segment (start 29.78 16.35) (end 46.35 22.555) (width 0.15) (layer "F.Cu") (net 29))
 (segment (start 29.78 18.89) (end 46.35 23.825) (width 0.15) (layer "F.Cu") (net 30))
 (segment (start 12 12.54) (end 29.78 18.89) (width 0.15) (layer "F.Cu") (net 30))
 (segment (start 29.78 21.43) (end 46.35 25.095) (width 0.15) (layer "F.Cu") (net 31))
 (segment (start 12 17.62) (end 29.78 21.43) (width 0.15) (layer "F.Cu") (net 31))
 (segment (start 12 20.16) (end 29.78 23.97) (width 0.15) (layer "F.Cu") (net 32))
 (segment (start 29.78 23.97) (end 46.35 26.365) (width 0.15) (layer "F.Cu") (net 32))
 (segment (start 29.78 26.51) (end 46.35 27.635) (width 0.15) (layer "F.Cu") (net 33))
 (segment (start 12 22.7) (end 29.78 26.51) (width 0.15) (layer "F.Cu") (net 33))
 (segment (start 12 25.24) (end 29.78 29.05) (width 0.15) (layer "F.Cu") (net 34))
 (segment (start 29.78 29.05) (end 46.35 28.905) (width 0.15) (layer "F.Cu") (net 34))
 (segment (start 12 30.32) (end 29.78 31.59) (width 0.15) (layer "F.Cu") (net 35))
 (segment (start 29.78 31.59) (end 46.35 30.175) (width 0.15) (layer "F.Cu") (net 35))
 (segment (start 29.78 34.13) (end 46.35 31.445) (width 0.15) (layer "F.Cu") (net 36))
 (segment (start 12 32.86) (end 29.78 34.13) (width 0.15) (layer "F.Cu") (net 36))
 (segment (start 46.35 47.555) (end 29.78 39.21) (width 0.15) (layer "F.Cu") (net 12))
 (segment (start 29.78 39.21) (end 12 35.4) (width 0.15) (layer "F.Cu") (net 12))
 (segment (start 29.78 41.75) (end 12 37.94) (width 0.15) (layer "F.Cu") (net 13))
 (segment (start 46.35 48.825) (end 29.78 41.75) (width 0.15) (layer "F.Cu") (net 13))
 (segment (start 46.35 50.095) (end 29.78 44.29) (width 0.15) (layer "F.Cu") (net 14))
 (segment (start 29.78 44.29) (end 12 43.02) (width 0.15) (layer "F.Cu") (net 14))
 (segment (start 29.78 46.83) (end 12 45.56) (width 0.15) (layer "F.Cu") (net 15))
 (segment (start 46.35 51.365) (end 29.78 46.83) (width 0.15) (layer "F.Cu") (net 15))
 (segment (start 29.78 49.37) (end 12 48.1) (width 0.15) (layer "F.Cu") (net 16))
 (segment (start 46.35 52.635) (end 29.78 49.37) (width 0.15) (layer "F.Cu") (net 16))
 (segment (start 46.35 53.905) (end 29.78 51.91) (width 0.15) (layer "F.Cu") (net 17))
 (segment (start 29.78 51.91) (end 12 50.64) (width 0.15) (layer "F.Cu") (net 17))
 (segment (start 46.35 55.175) (end 29.78 54.45) (width 0.15) (layer "F.Cu") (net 18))
 (segment (start 29.78 54.45) (end 12 55.72) (width 0.15) (layer "F.Cu") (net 18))
 (segment (start 29.78 56.99) (end 12 58.26) (width 0.15) (layer "F.Cu") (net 19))
 (segment (start 46.35 56.445) (end 29.78 56.99) (width 0.15) (layer "F.Cu") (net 19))
 (segment (start 55.65 23.825) (end 94 22.54) (width 0.25) (layer "F.Cu") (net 2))
 (segment (start 55.65 25.095) (end 94 25.08) (width 0.25) (layer "F.Cu") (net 3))
 (segment (start 55.65 26.365) (end 94 27.62) (width 0.25) (layer "F.Cu") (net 4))
 (segment (start 55.65 27.635) (end 94 30.16) (width 0.25) (layer "F.Cu") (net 5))
 (segment (start 55.65 28.905) (end 94 32.7) (width 0.25) (layer "F.Cu") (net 6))
 (segment (start 55.65 30.175) (end 94 35.24) (width 0.25) (layer "F.Cu") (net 7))
 (segment (start 55.65 31.445) (end 94 37.78) (width 0.25) (layer "F.Cu") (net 8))
 (segment (start 55.65 32.715) (end 94 40.32) (width 0.25) (layer "F.Cu") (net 9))
 (segment (start 94 49.54) (end 55.65 48.825) (width 0.25) (layer "F.Cu") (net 27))
 (segment (start 94 52.08) (end 55.65 50.095) (width 0.25) (layer "F.Cu") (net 26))
 (segment (start 94 54.62) (end 55.65 51.365) (width 0.25) (layer "F.Cu") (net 25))
 (segment (start 94 57.16) (end 55.65 52.635) (width 0.25) (layer "F.Cu") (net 24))
 (segment (start 94 59.7) (end 55.65 53.905) (width 0.25) (layer "F.Cu") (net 23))
 (segment (start 94 62.24) (end 55.65 55.175) (width 0.25) (layer "F.Cu") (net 22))
 (segment (start 94 64.78) (end 55.65 56.445) (width 0.25) (layer "F.Cu") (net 21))
 (segment (start 94 67.32) (end 55.65 57.715) (width 0.25) (layer "F.Cu") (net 20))
 (segment (start 63 22.555) (end 63 15) (width 0.25) (layer "F.Cu") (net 10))
 (segment (start 55.65 22.555) (end 63 22.555) (width 0.25) (layer "F.Cu") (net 10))
 (segment (start 57.5 22.555) (end 55.65 22.555) (width 0.25) (layer "F.Cu") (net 10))
 (segment (start 63 15) (end 62.0875 15) (width 0.25) (layer "F.Cu") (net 10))
 (via (at 57.5 22.555) (size 0.6) (drill 0.3) (layers "F.Cu" "B.Cu") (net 10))
 (segment (start 59 22.555) (end 57.5 22.555) (width 0.25) (layer "B.Cu") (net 10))
 (segment (start 59 58.26) (end 59 22.555) (width 0.25) (layer "B.Cu") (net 10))
 (segment (start 29.78 58.26) (end 59 58.26) (width 0.25) (layer "B.Cu") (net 10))
 (segment (start 57.5 47.555) (end 55.65 47.555) (width 0.25) (layer "F.Cu") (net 28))
 (segment (start 63 47.555) (end 63 40) (width 0.25) (layer "F.Cu") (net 28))
 (segment (start 63 40) (end 62.0875 40) (width 0.25) (layer "F.Cu") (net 28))
 (segment (start 55.65 47.555) (end 63 47.555) (width 0.25) (layer "F.Cu") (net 28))
 (via (at 57.5 47.555) (size 0.6) (drill 0.3) (layers "F.Cu" "B.Cu") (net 28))
 (segment (start 29.78 55.72) (end 57.5 47.555) (width 0.25) (layer "B.Cu") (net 28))
 (segment (start 29.78 32.86) (end 38.4 32.86) (width 0.25) (layer "B.Cu") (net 41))
 (segment (start 38.4 32.86) (end 38.4 10.62) (width 0.25) (layer "B.Cu") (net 41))
 (segment (start 38.4 10.62) (end 40 10.62) (width 0.25) (layer "B.Cu") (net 41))
 (segment (start 36.6 30.32) (end 36.6 8.08) (width 0.25) (layer "B.Cu") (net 40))
 (segment (start 29.78 30.32) (end 36.6 30.32) (width 0.25) (layer "B.Cu") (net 40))
 (segment (start 36.6 8.08) (end 40 8.08) (width 0.25) (layer "B.Cu") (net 40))
 (segment (start 29.78 25.24) (end 33 25.24) (width 0.25) (layer "B.Cu") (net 38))
 (segment (start 33 25.24) (end 33 3) (width 0.25) (layer "B.Cu") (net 38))
 (segment (start 33 3) (end 40 3) (width 0.25) (layer "B.Cu") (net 38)))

